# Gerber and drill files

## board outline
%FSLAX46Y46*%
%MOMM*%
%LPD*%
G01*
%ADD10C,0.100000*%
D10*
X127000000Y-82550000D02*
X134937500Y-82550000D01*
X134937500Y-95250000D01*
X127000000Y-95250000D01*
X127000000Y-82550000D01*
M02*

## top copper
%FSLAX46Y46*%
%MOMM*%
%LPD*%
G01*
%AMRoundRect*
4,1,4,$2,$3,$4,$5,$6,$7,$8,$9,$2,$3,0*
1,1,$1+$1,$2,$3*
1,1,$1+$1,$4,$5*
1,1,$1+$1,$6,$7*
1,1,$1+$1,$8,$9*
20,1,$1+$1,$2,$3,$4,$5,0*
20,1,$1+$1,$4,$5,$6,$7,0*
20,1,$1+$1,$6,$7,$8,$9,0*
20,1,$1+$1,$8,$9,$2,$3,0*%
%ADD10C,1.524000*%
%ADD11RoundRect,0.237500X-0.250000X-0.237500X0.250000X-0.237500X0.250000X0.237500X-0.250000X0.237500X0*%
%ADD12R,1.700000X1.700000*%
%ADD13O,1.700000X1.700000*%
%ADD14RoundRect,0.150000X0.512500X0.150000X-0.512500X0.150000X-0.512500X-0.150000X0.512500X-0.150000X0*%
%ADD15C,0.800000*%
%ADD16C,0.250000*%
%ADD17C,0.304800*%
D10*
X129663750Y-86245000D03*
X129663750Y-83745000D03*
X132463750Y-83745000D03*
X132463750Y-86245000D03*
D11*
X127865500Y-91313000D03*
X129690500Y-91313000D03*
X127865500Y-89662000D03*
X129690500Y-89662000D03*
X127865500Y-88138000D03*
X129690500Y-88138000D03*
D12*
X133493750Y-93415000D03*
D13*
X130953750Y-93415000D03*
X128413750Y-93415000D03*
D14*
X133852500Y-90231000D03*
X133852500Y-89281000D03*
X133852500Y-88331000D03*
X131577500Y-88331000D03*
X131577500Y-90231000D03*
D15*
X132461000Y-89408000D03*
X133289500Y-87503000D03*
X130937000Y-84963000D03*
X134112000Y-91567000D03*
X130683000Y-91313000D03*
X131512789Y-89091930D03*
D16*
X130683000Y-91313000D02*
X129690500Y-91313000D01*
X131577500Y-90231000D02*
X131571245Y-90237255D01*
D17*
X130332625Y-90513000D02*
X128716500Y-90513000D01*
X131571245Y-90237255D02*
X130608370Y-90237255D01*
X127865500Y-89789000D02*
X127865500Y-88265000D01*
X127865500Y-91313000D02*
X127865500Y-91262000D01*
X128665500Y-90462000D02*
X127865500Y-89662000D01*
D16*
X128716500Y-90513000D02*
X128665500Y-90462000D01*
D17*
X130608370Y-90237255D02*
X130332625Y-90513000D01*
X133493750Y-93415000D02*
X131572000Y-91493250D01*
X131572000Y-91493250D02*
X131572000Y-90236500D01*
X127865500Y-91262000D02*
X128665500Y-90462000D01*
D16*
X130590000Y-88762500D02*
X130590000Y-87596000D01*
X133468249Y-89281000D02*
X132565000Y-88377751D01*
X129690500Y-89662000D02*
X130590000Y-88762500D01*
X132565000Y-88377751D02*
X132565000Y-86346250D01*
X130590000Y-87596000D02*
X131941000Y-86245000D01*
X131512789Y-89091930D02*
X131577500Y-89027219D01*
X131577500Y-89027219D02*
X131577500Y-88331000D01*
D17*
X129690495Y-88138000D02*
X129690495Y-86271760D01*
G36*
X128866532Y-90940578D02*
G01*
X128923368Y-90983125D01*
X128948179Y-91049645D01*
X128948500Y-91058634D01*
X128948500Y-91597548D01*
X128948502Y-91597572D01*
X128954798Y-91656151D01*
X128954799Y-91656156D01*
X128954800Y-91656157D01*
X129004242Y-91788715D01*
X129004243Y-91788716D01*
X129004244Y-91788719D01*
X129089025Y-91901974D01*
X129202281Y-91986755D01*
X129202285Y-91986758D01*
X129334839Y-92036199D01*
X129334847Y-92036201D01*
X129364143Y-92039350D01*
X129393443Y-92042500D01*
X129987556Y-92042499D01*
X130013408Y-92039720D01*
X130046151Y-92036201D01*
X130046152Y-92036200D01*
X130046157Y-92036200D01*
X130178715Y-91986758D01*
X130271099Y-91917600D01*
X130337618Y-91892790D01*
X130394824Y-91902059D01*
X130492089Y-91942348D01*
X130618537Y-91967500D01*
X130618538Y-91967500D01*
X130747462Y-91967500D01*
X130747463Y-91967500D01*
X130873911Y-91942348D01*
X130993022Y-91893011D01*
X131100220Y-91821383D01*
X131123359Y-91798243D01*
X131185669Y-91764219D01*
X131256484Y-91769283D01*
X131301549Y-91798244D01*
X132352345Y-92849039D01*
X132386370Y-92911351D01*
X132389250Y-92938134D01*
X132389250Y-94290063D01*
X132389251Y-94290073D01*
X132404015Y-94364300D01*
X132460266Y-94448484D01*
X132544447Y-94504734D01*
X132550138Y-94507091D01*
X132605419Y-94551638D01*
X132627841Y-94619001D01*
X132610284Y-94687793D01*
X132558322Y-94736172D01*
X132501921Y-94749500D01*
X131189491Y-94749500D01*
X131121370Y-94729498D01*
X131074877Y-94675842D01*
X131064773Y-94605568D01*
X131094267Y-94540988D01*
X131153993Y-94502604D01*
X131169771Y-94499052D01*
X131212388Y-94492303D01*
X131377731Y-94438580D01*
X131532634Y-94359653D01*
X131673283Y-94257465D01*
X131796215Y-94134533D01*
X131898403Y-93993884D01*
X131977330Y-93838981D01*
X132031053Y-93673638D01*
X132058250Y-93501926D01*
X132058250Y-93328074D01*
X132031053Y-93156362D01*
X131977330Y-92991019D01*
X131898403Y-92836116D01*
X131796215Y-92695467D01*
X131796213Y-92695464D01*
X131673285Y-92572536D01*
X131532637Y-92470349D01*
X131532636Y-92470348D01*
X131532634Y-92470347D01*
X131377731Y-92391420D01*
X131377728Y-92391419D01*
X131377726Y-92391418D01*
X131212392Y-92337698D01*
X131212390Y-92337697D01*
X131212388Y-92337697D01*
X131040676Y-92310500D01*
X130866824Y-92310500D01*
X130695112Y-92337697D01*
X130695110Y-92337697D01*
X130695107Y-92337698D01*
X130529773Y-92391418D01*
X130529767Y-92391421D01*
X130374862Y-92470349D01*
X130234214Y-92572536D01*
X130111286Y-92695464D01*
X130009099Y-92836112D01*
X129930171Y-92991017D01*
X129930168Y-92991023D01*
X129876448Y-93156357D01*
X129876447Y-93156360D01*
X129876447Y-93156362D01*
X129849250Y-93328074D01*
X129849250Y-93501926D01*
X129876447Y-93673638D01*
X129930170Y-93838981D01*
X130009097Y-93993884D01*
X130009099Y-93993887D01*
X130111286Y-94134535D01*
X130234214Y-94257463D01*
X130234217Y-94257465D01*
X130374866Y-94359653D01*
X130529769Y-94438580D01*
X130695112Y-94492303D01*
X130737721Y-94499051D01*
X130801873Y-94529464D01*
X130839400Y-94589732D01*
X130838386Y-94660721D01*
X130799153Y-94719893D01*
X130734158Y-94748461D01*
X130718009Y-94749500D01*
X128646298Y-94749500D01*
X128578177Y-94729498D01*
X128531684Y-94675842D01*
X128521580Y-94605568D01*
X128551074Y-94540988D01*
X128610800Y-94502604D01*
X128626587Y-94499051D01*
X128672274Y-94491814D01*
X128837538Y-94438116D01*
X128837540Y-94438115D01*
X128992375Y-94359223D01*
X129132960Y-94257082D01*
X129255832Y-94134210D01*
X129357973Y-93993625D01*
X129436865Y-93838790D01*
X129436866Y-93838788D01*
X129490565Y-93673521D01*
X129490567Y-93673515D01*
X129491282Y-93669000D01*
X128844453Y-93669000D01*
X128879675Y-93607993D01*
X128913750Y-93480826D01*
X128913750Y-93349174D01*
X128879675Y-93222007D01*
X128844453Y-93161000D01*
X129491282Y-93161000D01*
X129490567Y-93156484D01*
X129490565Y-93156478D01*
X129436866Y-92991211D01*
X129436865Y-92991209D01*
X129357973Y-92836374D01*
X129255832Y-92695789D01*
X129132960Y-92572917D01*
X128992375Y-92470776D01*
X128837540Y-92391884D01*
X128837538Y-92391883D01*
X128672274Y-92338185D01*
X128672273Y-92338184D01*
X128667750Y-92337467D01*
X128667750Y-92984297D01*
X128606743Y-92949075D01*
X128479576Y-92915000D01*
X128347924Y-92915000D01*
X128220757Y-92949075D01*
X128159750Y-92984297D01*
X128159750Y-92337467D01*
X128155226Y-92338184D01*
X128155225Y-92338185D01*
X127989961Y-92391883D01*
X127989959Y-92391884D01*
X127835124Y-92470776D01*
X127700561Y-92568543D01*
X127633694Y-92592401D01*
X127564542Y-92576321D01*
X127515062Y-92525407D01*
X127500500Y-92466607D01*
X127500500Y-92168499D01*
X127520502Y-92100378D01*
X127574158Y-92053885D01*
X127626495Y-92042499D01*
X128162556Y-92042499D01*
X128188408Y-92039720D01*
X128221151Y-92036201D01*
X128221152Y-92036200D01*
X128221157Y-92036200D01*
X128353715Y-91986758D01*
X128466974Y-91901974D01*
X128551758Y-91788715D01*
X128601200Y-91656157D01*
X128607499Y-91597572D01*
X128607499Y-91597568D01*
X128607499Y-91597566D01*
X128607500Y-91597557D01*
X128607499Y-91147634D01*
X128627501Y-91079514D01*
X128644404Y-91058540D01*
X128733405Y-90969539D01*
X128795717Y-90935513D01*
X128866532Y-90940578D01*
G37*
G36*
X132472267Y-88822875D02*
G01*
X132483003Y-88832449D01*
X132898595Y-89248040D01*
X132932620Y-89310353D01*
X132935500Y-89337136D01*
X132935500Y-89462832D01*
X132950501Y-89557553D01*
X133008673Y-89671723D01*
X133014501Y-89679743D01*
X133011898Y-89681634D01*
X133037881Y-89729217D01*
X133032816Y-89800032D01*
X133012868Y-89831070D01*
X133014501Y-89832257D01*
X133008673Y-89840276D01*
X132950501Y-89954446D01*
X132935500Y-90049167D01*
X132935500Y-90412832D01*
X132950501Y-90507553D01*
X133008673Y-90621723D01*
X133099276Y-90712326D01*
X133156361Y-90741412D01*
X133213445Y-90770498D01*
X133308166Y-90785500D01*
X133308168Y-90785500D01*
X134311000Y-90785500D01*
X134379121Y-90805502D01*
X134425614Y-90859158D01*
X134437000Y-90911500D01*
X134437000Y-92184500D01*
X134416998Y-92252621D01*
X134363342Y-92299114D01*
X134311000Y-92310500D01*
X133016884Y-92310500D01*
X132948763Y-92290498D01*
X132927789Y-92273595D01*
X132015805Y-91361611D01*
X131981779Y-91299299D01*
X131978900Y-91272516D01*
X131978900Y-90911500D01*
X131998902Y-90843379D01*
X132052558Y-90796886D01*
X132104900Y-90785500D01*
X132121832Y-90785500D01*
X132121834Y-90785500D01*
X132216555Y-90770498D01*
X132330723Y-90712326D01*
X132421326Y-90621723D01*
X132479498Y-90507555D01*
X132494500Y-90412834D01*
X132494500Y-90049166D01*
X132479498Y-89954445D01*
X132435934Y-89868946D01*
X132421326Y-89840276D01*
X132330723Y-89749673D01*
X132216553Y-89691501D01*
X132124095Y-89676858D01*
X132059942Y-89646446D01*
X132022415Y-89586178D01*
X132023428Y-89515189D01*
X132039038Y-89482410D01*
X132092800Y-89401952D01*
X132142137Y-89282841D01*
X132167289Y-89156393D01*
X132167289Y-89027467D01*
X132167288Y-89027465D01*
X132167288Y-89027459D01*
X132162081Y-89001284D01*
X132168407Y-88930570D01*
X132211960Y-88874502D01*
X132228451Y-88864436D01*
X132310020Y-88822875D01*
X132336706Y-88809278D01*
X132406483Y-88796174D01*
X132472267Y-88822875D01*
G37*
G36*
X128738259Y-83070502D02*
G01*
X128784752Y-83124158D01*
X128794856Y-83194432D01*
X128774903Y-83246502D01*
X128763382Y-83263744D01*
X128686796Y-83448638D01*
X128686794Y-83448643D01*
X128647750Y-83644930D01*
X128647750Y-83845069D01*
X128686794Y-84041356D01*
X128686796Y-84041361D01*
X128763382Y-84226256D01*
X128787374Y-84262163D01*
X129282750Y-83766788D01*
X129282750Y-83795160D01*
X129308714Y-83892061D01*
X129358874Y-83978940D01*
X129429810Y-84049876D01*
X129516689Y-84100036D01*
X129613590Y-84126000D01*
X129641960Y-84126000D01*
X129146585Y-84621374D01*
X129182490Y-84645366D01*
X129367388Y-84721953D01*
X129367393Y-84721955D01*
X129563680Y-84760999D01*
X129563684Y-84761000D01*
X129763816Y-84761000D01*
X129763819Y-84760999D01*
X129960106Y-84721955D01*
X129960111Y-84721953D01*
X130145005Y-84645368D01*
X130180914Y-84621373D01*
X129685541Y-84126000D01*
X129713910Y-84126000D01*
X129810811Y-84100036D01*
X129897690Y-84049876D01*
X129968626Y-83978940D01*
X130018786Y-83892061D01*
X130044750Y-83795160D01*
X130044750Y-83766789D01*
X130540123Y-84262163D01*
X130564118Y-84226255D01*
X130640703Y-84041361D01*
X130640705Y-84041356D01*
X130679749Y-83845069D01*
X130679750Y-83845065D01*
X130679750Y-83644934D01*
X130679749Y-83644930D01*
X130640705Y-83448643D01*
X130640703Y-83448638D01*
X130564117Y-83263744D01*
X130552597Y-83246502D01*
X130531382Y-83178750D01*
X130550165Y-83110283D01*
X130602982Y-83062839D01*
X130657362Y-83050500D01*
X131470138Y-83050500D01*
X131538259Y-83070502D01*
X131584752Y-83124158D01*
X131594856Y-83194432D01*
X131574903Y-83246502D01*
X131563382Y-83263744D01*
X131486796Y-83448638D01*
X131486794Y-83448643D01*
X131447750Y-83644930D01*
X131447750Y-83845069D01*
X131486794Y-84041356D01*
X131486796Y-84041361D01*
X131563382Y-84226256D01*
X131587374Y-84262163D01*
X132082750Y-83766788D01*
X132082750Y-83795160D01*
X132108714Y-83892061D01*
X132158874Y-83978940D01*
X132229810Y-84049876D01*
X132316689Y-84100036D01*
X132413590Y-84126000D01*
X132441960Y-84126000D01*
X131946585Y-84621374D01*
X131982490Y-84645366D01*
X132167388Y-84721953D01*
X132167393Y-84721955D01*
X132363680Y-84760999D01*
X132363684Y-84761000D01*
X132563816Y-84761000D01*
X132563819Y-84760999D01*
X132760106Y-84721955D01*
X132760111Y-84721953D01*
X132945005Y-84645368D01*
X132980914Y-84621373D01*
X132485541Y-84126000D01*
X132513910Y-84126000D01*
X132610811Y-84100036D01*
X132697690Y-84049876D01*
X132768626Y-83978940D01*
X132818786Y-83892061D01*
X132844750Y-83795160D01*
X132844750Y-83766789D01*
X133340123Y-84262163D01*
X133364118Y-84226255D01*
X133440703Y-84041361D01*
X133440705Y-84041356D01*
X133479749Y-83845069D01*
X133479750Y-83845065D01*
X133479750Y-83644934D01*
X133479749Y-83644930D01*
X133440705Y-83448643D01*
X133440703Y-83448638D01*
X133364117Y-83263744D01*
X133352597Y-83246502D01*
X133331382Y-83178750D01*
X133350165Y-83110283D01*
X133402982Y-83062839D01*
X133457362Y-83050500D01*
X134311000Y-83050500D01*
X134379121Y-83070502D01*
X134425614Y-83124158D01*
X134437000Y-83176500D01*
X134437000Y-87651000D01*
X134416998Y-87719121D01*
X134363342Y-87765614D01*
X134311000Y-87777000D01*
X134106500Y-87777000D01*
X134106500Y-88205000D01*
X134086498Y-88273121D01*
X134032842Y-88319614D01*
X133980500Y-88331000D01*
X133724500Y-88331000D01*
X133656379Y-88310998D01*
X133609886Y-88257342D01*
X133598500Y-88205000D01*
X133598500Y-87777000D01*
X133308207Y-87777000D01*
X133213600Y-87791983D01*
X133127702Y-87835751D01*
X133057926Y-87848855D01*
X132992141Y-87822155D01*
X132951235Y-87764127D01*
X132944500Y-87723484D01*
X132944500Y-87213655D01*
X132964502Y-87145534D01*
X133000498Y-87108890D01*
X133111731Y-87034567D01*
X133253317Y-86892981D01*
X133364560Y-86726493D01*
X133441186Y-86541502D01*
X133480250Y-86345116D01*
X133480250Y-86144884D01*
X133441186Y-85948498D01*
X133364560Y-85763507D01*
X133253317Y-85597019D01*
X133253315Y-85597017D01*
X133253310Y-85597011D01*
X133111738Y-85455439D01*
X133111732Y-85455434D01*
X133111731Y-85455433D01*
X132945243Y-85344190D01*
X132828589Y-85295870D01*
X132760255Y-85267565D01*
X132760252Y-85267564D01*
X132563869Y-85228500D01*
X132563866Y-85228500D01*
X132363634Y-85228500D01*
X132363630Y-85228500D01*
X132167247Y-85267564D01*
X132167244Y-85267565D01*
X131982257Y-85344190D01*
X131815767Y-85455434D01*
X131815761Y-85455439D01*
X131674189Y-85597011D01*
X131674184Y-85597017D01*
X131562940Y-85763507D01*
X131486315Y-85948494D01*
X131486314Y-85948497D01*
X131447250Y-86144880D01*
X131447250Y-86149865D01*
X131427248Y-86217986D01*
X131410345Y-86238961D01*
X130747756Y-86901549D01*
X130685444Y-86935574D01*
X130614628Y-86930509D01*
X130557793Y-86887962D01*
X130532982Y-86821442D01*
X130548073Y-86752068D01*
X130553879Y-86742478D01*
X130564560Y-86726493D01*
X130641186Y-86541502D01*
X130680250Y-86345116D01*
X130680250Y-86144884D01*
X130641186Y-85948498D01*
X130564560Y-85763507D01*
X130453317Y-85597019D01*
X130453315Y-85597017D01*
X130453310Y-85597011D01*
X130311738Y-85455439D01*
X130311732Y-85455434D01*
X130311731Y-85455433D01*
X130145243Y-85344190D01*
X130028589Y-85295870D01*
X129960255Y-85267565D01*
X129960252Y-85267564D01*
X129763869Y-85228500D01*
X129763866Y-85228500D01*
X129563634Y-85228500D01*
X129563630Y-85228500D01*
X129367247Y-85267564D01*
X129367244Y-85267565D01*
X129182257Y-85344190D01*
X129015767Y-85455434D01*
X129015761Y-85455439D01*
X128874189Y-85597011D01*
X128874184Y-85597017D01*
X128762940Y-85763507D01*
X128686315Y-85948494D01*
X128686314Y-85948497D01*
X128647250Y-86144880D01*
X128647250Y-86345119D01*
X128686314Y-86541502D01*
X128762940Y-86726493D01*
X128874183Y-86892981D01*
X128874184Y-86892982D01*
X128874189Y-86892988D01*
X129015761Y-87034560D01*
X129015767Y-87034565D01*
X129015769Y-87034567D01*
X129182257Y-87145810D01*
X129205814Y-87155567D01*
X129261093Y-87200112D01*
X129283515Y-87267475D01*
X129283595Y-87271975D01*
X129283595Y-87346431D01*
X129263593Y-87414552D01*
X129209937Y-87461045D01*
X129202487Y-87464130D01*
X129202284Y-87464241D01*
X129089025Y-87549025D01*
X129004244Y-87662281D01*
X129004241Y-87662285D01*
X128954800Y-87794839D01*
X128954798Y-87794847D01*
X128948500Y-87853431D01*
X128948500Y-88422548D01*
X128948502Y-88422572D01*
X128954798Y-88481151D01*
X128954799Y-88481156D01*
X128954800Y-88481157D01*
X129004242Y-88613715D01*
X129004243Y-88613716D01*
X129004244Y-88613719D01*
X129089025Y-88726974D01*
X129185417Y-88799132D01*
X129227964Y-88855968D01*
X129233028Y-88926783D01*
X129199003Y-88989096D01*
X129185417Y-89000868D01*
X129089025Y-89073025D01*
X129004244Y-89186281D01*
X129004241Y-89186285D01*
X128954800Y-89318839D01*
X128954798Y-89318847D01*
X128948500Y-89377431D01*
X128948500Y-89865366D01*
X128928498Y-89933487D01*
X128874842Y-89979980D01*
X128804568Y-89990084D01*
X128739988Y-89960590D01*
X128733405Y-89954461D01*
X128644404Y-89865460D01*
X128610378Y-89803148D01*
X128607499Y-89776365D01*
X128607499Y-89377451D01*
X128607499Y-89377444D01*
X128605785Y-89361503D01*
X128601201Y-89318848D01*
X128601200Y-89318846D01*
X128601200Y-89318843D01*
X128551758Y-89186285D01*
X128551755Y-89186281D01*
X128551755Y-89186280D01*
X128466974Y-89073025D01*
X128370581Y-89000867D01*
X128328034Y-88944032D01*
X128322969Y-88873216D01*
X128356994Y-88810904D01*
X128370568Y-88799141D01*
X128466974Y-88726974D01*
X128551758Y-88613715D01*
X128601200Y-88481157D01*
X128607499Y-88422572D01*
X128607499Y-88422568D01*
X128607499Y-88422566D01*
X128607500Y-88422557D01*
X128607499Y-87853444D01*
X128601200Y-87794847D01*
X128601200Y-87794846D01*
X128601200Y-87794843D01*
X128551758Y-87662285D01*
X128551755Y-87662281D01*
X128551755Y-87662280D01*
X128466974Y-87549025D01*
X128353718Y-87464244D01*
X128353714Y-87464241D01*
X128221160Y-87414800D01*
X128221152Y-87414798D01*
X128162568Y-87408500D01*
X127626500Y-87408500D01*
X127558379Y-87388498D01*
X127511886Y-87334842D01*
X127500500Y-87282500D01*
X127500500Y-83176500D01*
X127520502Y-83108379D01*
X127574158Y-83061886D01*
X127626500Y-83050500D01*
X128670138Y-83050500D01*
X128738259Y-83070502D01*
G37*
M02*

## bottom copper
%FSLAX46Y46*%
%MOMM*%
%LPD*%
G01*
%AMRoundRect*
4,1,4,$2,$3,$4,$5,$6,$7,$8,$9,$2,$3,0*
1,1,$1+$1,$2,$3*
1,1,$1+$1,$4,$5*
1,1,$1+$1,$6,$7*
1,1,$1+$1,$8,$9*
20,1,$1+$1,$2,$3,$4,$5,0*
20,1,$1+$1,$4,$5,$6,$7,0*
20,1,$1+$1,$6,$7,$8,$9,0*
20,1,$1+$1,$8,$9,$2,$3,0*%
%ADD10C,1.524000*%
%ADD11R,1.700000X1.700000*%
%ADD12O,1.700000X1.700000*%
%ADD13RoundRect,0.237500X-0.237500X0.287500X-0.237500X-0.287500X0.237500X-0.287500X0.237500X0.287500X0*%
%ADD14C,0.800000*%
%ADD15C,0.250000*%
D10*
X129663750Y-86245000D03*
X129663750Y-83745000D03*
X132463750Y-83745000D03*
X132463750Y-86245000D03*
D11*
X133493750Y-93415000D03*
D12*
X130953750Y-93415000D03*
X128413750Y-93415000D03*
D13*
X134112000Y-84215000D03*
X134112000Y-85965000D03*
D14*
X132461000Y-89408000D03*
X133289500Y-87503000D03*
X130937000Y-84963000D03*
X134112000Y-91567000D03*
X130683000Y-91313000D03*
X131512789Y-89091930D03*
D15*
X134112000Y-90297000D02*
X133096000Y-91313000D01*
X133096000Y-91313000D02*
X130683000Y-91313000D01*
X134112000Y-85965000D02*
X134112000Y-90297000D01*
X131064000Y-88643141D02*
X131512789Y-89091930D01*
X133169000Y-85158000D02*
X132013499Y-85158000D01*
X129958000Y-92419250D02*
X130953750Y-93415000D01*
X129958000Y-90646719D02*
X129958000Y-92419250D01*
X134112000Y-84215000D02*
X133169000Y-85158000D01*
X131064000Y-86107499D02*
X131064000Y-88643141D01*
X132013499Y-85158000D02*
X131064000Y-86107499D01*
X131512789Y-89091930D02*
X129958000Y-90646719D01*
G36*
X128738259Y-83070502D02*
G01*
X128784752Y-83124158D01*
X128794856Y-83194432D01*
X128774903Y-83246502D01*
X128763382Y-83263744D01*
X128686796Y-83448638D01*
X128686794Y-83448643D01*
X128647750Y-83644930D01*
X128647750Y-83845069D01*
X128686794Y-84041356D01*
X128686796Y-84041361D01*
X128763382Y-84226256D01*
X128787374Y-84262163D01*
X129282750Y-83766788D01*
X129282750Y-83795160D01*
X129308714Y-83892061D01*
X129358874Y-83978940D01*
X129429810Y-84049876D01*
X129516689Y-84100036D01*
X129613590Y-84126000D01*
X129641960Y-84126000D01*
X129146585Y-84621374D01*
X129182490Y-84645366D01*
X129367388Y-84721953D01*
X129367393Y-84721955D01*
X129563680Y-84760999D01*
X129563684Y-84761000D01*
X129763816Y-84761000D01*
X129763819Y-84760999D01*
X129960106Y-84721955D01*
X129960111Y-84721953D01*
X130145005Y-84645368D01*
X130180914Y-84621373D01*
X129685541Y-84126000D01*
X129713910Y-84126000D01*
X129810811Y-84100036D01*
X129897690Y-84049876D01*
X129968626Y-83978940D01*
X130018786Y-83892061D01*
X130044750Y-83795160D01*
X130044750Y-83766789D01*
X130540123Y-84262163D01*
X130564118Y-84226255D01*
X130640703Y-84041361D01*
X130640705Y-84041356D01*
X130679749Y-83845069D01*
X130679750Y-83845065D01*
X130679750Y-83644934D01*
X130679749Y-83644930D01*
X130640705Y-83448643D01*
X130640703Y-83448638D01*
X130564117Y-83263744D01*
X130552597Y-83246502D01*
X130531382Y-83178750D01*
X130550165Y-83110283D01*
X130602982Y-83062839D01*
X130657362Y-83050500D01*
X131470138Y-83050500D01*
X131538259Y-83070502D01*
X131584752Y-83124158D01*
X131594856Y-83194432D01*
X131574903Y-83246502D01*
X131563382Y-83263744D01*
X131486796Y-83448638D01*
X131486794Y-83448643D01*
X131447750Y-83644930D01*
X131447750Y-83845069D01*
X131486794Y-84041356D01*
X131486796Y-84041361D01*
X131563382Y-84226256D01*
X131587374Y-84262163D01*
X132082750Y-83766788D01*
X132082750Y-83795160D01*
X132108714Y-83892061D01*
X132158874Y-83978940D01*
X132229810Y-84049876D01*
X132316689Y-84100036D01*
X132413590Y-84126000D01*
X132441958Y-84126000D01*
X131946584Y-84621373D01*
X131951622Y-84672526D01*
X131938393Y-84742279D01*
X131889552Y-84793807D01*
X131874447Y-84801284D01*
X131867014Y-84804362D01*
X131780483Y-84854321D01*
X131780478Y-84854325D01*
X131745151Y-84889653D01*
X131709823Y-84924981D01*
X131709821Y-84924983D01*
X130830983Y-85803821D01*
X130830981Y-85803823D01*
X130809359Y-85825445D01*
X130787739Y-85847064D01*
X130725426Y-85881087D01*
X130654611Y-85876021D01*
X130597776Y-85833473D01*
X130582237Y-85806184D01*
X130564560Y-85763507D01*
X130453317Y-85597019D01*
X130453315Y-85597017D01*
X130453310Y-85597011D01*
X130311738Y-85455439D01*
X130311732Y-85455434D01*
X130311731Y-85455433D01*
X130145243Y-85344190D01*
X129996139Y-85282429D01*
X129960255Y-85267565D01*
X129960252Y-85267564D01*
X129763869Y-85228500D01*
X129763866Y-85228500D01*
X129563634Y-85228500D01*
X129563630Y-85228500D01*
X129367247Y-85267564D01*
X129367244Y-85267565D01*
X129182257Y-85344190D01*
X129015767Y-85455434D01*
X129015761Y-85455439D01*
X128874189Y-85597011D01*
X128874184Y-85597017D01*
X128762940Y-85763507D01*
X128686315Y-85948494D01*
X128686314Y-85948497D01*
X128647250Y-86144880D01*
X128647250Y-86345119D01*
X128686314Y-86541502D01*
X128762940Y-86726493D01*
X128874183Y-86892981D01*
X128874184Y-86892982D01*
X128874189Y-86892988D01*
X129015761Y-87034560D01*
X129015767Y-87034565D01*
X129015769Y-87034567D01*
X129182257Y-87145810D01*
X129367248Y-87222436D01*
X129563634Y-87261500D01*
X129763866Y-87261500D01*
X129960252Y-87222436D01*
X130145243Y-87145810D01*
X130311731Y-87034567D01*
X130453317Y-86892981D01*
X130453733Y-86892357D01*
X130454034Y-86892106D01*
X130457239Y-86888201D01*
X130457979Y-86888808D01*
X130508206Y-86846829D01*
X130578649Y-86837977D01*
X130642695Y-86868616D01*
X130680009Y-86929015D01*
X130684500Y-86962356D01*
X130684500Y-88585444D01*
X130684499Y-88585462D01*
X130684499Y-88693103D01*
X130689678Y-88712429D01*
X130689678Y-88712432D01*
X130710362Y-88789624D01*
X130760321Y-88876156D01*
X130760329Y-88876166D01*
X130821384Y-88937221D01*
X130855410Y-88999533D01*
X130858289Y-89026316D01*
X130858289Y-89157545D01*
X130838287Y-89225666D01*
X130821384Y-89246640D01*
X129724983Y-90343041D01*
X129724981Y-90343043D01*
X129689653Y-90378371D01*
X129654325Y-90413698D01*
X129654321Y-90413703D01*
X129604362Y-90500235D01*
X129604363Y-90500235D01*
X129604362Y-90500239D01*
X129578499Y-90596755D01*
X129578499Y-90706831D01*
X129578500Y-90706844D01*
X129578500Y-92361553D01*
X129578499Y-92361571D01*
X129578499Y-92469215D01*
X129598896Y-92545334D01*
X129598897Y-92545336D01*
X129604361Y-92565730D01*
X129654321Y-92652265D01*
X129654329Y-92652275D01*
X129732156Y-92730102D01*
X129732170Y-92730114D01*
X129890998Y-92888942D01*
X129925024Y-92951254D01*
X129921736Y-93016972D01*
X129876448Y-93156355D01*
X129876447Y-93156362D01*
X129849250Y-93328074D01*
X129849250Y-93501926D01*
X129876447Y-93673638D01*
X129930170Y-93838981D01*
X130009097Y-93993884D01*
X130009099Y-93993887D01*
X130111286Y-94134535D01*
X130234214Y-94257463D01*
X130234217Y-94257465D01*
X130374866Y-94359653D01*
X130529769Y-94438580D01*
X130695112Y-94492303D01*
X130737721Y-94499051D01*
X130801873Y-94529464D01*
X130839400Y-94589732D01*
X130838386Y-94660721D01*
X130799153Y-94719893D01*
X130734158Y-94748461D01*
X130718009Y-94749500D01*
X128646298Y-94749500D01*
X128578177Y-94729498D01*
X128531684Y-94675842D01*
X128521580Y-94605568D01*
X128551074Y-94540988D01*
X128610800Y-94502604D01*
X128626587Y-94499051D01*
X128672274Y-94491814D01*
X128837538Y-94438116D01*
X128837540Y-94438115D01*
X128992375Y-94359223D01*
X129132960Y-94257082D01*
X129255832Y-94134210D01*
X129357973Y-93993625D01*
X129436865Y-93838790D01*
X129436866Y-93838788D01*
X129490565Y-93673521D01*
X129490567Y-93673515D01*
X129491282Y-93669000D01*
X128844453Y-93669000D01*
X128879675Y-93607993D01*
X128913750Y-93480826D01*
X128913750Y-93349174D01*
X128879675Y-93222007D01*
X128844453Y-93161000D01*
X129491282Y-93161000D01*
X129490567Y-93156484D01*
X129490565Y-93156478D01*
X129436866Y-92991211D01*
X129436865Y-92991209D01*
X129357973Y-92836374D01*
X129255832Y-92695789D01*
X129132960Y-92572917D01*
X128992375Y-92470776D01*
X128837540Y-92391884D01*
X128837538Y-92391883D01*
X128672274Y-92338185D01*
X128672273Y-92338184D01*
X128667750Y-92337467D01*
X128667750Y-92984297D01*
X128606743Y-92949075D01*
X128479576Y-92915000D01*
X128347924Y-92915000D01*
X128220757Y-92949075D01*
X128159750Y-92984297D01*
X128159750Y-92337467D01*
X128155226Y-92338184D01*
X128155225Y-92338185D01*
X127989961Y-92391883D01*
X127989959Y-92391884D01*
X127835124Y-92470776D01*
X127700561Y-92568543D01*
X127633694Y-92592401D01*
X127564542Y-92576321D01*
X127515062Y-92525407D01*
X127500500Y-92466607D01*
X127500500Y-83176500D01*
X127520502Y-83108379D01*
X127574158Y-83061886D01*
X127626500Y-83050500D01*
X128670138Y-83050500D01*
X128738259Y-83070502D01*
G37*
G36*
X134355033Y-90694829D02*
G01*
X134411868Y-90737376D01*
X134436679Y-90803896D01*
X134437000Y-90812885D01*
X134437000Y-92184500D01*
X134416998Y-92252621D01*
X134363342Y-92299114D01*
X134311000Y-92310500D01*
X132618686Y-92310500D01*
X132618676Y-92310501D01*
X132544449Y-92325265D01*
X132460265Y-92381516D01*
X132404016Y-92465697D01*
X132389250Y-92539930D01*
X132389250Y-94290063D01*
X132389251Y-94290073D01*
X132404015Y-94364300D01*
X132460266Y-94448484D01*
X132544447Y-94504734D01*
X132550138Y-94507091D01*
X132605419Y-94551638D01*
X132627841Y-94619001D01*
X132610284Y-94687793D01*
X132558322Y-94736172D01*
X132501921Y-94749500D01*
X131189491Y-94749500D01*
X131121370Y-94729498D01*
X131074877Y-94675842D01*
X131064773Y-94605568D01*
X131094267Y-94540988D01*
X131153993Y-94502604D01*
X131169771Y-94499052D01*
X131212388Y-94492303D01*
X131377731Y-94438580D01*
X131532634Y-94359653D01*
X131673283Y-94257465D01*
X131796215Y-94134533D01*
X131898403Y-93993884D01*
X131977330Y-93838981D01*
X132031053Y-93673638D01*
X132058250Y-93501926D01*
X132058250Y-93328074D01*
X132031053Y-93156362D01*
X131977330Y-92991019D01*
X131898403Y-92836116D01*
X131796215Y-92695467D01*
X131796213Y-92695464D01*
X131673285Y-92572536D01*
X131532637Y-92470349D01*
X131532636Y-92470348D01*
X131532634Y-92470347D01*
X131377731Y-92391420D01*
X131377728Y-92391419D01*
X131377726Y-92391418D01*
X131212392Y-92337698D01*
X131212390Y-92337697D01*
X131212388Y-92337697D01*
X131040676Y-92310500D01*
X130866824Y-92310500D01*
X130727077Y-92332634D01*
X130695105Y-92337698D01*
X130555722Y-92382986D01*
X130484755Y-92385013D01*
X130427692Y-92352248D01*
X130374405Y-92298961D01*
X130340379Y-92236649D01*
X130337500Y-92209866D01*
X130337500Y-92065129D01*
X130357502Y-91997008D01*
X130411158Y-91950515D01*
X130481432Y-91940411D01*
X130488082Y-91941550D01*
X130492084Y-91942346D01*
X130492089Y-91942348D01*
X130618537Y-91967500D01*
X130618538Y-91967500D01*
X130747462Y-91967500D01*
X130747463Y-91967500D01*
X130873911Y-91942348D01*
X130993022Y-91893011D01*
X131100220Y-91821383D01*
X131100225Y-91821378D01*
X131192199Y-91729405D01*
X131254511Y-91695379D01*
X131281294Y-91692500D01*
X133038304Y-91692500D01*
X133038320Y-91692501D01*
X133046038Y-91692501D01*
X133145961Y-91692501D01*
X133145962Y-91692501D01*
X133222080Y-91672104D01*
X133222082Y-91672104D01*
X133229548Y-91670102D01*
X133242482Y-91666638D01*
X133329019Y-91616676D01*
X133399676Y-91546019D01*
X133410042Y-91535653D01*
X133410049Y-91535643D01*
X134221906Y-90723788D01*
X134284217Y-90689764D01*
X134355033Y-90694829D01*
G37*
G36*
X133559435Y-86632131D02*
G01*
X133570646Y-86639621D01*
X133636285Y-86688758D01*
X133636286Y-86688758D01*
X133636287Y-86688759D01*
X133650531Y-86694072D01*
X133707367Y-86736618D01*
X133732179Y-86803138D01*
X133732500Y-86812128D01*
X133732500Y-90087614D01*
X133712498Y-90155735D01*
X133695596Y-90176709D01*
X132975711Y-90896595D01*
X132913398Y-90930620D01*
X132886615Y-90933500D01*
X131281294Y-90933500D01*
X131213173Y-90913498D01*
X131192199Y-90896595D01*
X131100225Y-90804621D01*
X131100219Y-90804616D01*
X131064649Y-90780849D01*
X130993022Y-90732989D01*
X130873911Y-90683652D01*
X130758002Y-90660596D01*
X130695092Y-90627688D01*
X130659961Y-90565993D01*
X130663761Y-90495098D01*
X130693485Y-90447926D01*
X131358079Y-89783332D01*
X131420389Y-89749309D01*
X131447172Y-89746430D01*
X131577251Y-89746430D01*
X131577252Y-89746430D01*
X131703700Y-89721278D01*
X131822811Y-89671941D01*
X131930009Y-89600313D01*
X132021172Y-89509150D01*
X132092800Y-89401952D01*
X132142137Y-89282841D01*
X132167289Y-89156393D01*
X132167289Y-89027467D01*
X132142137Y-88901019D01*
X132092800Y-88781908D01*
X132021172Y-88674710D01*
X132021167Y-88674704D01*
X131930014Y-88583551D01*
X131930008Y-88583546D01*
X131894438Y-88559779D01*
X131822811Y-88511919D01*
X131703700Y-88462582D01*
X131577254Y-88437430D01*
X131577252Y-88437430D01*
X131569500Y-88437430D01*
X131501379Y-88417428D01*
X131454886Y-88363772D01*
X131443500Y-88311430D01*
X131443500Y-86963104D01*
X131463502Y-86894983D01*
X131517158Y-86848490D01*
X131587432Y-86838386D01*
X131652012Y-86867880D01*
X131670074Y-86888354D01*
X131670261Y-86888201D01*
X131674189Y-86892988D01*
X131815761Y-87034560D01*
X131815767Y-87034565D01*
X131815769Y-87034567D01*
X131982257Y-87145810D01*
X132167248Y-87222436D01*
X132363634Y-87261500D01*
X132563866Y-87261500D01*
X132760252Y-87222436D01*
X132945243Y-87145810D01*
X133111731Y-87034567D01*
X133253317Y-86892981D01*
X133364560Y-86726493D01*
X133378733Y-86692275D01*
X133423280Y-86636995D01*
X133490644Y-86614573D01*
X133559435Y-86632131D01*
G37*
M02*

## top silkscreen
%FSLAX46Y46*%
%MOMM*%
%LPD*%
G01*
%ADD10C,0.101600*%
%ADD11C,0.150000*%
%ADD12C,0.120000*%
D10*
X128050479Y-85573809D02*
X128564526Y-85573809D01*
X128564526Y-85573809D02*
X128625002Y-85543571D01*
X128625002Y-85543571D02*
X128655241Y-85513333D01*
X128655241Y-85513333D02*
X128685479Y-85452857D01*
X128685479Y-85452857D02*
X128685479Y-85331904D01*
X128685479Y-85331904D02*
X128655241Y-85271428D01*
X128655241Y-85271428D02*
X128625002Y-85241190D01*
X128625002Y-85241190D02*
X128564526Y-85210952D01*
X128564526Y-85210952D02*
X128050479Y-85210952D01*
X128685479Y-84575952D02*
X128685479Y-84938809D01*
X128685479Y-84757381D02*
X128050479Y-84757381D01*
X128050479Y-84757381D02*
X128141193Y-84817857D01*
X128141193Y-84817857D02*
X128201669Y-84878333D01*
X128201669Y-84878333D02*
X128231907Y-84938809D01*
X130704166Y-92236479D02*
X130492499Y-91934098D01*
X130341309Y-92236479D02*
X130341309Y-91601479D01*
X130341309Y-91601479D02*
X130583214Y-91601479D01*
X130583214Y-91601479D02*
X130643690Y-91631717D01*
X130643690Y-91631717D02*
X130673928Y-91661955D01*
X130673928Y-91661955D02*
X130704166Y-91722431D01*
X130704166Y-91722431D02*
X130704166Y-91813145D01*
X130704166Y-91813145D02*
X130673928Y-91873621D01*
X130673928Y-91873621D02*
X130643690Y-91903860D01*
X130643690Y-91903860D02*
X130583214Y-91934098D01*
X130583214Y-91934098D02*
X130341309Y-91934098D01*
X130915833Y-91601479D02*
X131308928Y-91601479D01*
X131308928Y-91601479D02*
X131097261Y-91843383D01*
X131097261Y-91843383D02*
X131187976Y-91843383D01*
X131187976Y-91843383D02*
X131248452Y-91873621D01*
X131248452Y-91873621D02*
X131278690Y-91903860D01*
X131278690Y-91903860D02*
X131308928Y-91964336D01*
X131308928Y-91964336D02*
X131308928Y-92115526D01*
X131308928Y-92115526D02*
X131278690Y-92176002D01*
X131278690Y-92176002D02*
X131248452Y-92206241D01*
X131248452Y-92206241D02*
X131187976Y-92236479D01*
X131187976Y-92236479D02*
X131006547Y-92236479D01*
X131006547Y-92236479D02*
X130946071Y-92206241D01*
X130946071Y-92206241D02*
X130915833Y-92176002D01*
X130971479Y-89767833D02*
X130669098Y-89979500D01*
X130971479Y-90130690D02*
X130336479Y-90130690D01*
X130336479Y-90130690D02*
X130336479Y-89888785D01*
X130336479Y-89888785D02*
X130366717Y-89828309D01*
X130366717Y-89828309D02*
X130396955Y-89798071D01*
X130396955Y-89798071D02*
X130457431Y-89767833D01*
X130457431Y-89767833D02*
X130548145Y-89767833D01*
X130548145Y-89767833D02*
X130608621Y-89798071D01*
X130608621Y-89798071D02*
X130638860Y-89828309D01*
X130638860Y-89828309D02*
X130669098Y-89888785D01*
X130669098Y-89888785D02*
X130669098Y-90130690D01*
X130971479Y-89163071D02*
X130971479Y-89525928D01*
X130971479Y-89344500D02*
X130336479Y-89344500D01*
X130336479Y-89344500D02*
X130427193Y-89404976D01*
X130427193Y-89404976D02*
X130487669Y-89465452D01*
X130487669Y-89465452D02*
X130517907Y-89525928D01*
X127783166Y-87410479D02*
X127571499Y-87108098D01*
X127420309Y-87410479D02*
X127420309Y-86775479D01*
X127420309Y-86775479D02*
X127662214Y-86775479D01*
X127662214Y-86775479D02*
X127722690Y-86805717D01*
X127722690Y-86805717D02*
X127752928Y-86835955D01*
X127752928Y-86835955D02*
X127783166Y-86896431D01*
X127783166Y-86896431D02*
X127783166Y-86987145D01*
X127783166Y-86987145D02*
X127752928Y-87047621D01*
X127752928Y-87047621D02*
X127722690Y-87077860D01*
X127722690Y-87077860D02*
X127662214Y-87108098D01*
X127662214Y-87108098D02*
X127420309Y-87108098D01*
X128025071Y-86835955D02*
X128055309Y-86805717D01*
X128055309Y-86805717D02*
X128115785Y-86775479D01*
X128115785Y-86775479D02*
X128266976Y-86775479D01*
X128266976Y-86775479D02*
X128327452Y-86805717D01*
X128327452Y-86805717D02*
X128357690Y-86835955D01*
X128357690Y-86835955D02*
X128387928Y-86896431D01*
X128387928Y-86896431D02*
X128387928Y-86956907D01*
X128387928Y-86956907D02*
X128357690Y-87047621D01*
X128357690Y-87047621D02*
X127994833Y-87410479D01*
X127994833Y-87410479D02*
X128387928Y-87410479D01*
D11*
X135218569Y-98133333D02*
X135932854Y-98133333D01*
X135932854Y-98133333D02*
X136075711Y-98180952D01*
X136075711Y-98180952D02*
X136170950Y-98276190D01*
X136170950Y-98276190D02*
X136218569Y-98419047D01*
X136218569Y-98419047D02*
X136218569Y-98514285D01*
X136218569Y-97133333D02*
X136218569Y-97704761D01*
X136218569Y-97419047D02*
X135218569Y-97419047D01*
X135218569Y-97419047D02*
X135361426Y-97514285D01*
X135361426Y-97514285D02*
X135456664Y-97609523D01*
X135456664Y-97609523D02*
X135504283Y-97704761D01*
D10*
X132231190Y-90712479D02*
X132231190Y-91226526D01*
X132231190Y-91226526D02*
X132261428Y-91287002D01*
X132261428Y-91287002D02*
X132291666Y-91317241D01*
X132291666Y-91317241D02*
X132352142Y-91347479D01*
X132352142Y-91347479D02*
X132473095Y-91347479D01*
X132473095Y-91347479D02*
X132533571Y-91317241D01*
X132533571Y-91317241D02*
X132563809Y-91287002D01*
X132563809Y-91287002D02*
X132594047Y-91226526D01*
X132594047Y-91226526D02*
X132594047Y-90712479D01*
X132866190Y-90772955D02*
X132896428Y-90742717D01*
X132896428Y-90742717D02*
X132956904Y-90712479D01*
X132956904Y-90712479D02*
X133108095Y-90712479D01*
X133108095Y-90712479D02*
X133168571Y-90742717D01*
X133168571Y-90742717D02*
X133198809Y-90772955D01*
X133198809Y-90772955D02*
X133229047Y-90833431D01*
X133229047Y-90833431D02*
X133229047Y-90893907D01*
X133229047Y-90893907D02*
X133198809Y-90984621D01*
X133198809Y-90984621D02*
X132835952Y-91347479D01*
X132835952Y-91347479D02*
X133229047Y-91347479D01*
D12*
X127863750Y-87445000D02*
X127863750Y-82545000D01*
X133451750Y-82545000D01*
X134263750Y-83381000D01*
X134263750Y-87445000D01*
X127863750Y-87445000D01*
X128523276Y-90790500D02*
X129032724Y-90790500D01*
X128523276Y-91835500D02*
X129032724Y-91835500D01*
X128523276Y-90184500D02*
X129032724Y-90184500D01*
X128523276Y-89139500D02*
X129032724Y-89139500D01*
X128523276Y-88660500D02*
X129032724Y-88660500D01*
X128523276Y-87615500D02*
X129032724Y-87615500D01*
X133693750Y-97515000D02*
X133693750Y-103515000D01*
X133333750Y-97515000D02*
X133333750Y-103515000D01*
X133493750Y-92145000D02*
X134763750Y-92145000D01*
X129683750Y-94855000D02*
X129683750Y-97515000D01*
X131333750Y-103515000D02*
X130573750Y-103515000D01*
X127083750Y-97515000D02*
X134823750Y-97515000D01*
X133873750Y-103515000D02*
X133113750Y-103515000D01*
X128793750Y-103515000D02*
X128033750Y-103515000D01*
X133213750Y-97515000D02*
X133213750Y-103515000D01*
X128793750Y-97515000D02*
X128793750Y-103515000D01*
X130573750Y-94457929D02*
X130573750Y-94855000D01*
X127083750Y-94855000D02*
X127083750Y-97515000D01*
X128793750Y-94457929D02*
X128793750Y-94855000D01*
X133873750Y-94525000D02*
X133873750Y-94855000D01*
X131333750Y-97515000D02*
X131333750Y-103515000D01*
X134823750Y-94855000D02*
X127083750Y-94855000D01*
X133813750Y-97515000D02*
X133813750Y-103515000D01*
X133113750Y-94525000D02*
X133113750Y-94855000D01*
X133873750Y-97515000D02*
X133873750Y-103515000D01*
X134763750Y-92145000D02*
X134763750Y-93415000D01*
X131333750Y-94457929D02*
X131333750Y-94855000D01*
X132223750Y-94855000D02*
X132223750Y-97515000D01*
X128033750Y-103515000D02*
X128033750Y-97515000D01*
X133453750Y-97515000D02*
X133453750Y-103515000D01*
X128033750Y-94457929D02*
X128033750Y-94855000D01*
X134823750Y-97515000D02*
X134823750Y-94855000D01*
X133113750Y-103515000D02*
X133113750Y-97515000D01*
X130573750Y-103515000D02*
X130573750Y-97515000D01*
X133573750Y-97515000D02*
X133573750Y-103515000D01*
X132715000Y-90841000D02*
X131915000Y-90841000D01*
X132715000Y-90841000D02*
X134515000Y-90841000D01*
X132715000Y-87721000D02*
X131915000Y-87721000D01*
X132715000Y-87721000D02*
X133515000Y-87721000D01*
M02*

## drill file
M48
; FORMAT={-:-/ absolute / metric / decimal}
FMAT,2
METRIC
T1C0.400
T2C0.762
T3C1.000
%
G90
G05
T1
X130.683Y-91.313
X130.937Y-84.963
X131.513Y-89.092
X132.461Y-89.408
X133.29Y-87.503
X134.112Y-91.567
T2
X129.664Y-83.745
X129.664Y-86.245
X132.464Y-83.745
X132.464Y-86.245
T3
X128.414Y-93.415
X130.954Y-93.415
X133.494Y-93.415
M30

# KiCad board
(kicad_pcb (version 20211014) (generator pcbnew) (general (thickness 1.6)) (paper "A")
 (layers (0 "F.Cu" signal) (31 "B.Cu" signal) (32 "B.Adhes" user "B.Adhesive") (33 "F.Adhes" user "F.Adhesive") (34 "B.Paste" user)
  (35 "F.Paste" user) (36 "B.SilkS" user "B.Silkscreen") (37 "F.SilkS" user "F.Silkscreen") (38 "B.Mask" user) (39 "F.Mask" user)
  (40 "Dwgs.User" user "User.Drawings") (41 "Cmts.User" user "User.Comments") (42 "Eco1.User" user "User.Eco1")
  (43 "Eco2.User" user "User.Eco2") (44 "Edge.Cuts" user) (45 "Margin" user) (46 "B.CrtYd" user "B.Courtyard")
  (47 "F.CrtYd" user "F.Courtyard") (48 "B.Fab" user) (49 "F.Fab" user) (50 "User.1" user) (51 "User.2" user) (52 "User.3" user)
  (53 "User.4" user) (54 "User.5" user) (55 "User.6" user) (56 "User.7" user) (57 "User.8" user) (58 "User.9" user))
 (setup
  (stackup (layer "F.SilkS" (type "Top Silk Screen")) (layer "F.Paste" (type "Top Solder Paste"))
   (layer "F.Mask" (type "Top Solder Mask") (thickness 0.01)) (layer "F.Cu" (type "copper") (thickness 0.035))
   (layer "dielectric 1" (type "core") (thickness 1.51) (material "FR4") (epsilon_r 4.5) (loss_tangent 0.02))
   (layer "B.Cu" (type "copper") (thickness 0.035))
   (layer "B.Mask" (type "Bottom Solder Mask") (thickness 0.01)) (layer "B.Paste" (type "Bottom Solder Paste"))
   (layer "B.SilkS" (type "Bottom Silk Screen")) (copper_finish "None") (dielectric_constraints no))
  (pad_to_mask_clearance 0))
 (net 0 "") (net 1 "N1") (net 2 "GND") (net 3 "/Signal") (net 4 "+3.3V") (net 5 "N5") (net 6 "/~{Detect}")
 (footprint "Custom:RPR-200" (layer "F.Cu") (at 127.86375 87.445)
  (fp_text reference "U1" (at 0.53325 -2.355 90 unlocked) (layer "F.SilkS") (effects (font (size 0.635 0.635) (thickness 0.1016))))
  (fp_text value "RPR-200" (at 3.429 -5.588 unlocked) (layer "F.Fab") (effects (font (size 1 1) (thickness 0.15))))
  (fp_poly (pts (xy 0 0) (xy 0 -4.9) (xy 5.588 -4.9) (xy 6.4 -4.064) (xy 6.4 0)) (layer "F.SilkS") (width 0.12) (fill none))
  (pad "1" thru_hole circle (at 1.8 -1.2) (size 1.524 1.524) (drill 0.762) (layers *.Cu *.Mask) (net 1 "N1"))
  (pad "2" thru_hole circle (at 1.8 -3.7) (size 1.524 1.524) (drill 0.762) (layers *.Cu *.Mask) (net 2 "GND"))
  (pad "3" thru_hole circle (at 4.6 -3.7) (size 1.524 1.524) (drill 0.762) (layers *.Cu *.Mask) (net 2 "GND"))
  (pad "4" thru_hole circle (at 4.6 -1.2) (size 1.524 1.524) (drill 0.762) (layers *.Cu *.Mask) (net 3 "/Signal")))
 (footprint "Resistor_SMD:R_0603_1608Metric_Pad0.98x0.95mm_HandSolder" (layer "F.Cu") (at 128.778 91.313)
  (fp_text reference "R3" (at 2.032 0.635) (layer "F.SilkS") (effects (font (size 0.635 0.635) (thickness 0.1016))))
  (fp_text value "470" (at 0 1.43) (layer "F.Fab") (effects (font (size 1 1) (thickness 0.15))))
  (fp_line (start -0.254724 -0.5225) (end 0.254724 -0.5225) (layer "F.SilkS") (width 0.12))
  (fp_line (start -0.254724 0.5225) (end 0.254724 0.5225) (layer "F.SilkS") (width 0.12))
  (pad "1" smd roundrect (at -0.9125 0) (size 0.975 0.95) (layers "F.Cu" "F.Paste" "F.Mask") (roundrect_rratio 0.25) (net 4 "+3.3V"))
  (pad "2" smd roundrect (at 0.9125 0) (size 0.975 0.95) (layers "F.Cu" "F.Paste" "F.Mask") (roundrect_rratio 0.25) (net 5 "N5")))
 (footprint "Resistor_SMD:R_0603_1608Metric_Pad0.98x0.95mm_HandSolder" (layer "F.Cu") (at 128.778 89.662)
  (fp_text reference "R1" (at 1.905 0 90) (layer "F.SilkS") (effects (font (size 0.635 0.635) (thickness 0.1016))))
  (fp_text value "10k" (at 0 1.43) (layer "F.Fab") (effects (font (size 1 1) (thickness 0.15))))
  (fp_line (start -0.254724 0.5225) (end 0.254724 0.5225) (layer "F.SilkS") (width 0.12))
  (fp_line (start -0.254724 -0.5225) (end 0.254724 -0.5225) (layer "F.SilkS") (width 0.12))
  (pad "1" smd roundrect (at -0.9125 0) (size 0.975 0.95) (layers "F.Cu" "F.Paste" "F.Mask") (roundrect_rratio 0.25) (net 4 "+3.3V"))
  (pad "2" smd roundrect (at 0.9125 0) (size 0.975 0.95) (layers "F.Cu" "F.Paste" "F.Mask") (roundrect_rratio 0.25) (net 3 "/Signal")))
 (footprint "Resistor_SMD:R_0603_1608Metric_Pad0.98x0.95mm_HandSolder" (layer "F.Cu") (at 128.778 88.138)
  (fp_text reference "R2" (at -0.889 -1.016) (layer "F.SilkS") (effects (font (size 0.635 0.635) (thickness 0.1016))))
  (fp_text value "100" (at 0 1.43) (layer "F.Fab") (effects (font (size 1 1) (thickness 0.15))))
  (fp_line (start -0.254724 0.5225) (end 0.254724 0.5225) (layer "F.SilkS") (width 0.12))
  (fp_line (start -0.254724 -0.5225) (end 0.254724 -0.5225) (layer "F.SilkS") (width 0.12))
  (pad "1" smd roundrect (at -0.9125 0) (size 0.975 0.95) (layers "F.Cu" "F.Paste" "F.Mask") (roundrect_rratio 0.25) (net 4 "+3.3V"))
  (pad "2" smd roundrect (at 0.9125 0) (size 0.975 0.95) (layers "F.Cu" "F.Paste" "F.Mask") (roundrect_rratio 0.25) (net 1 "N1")))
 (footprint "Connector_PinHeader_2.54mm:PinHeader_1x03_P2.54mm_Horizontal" (layer "F.Cu") (at 133.49375 93.415 -90)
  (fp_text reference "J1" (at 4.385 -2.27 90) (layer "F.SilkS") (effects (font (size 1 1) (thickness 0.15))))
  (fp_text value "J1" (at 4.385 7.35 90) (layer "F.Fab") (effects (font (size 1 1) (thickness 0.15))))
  (fp_line (start 4.1 -0.2) (end 10.1 -0.2) (layer "F.SilkS") (width 0.12))
  (fp_line (start 4.1 0.16) (end 10.1 0.16) (layer "F.SilkS") (width 0.12))
  (fp_line (start -1.27 0) (end -1.27 -1.27) (layer "F.SilkS") (width 0.12))
  (fp_line (start 1.44 3.81) (end 4.1 3.81) (layer "F.SilkS") (width 0.12))
  (fp_line (start 10.1 2.16) (end 10.1 2.92) (layer "F.SilkS") (width 0.12))
  (fp_line (start 4.1 6.41) (end 4.1 -1.33) (layer "F.SilkS") (width 0.12))
  (fp_line (start 10.1 -0.38) (end 10.1 0.38) (layer "F.SilkS") (width 0.12))
  (fp_line (start 10.1 4.7) (end 10.1 5.46) (layer "F.SilkS") (width 0.12))
  (fp_line (start 4.1 0.28) (end 10.1 0.28) (layer "F.SilkS") (width 0.12))
  (fp_line (start 4.1 4.7) (end 10.1 4.7) (layer "F.SilkS") (width 0.12))
  (fp_line (start 1.042929 2.92) (end 1.44 2.92) (layer "F.SilkS") (width 0.12))
  (fp_line (start 1.44 6.41) (end 4.1 6.41) (layer "F.SilkS") (width 0.12))
  (fp_line (start 1.042929 4.7) (end 1.44 4.7) (layer "F.SilkS") (width 0.12))
  (fp_line (start 1.11 -0.38) (end 1.44 -0.38) (layer "F.SilkS") (width 0.12))
  (fp_line (start 4.1 2.16) (end 10.1 2.16) (layer "F.SilkS") (width 0.12))
  (fp_line (start 1.44 -1.33) (end 1.44 6.41) (layer "F.SilkS") (width 0.12))
  (fp_line (start 4.1 -0.32) (end 10.1 -0.32) (layer "F.SilkS") (width 0.12))
  (fp_line (start 1.11 0.38) (end 1.44 0.38) (layer "F.SilkS") (width 0.12))
  (fp_line (start 4.1 -0.38) (end 10.1 -0.38) (layer "F.SilkS") (width 0.12))
  (fp_line (start -1.27 -1.27) (end 0 -1.27) (layer "F.SilkS") (width 0.12))
  (fp_line (start 1.042929 2.16) (end 1.44 2.16) (layer "F.SilkS") (width 0.12))
  (fp_line (start 1.44 1.27) (end 4.1 1.27) (layer "F.SilkS") (width 0.12))
  (fp_line (start 10.1 5.46) (end 4.1 5.46) (layer "F.SilkS") (width 0.12))
  (fp_line (start 4.1 0.04) (end 10.1 0.04) (layer "F.SilkS") (width 0.12))
  (fp_line (start 1.042929 5.46) (end 1.44 5.46) (layer "F.SilkS") (width 0.12))
  (fp_line (start 4.1 -1.33) (end 1.44 -1.33) (layer "F.SilkS") (width 0.12))
  (fp_line (start 10.1 0.38) (end 4.1 0.38) (layer "F.SilkS") (width 0.12))
  (fp_line (start 10.1 2.92) (end 4.1 2.92) (layer "F.SilkS") (width 0.12))
  (fp_line (start 4.1 -0.08) (end 10.1 -0.08) (layer "F.SilkS") (width 0.12))
  (pad "1" thru_hole rect (at 0 0 270) (size 1.7 1.7) (drill 1) (layers *.Cu *.Mask) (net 4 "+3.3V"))
  (pad "2" thru_hole oval (at 0 2.54 270) (size 1.7 1.7) (drill 1) (layers *.Cu *.Mask) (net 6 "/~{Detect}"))
  (pad "3" thru_hole oval (at 0 5.08 270) (size 1.7 1.7) (drill 1) (layers *.Cu *.Mask) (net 2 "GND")))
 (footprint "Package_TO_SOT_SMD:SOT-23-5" (layer "F.Cu") (at 132.715 89.281 180)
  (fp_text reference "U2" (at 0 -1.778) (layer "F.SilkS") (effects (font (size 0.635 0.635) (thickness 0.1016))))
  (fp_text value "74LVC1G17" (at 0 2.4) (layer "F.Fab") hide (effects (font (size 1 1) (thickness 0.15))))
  (fp_line (start 0 -1.56) (end 0.8 -1.56) (layer "F.SilkS") (width 0.12))
  (fp_line (start 0 -1.56) (end -1.8 -1.56) (layer "F.SilkS") (width 0.12))
  (fp_line (start 0 1.56) (end 0.8 1.56) (layer "F.SilkS") (width 0.12))
  (fp_line (start 0 1.56) (end -0.8 1.56) (layer "F.SilkS") (width 0.12))
  (pad "1" smd roundrect (at -1.1375 -0.95 180) (size 1.325 0.6) (layers "F.Cu" "F.Paste" "F.Mask") (roundrect_rratio 0.25))
  (pad "2" smd roundrect (at -1.1375 0 180) (size 1.325 0.6) (layers "F.Cu" "F.Paste" "F.Mask") (roundrect_rratio 0.25) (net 3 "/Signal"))
  (pad "3" smd roundrect (at -1.1375 0.95 180) (size 1.325 0.6) (layers "F.Cu" "F.Paste" "F.Mask") (roundrect_rratio 0.25) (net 2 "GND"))
  (pad "4" smd roundrect (at 1.1375 0.95 180) (size 1.325 0.6) (layers "F.Cu" "F.Paste" "F.Mask") (roundrect_rratio 0.25)
   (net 6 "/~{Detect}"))
  (pad "5" smd roundrect (at 1.1375 -0.95 180) (size 1.325 0.6) (layers "F.Cu" "F.Paste" "F.Mask") (roundrect_rratio 0.25) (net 4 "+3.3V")))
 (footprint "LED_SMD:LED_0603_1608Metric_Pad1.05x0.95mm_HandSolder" (layer "B.Cu") (at 134.112 85.09 -90)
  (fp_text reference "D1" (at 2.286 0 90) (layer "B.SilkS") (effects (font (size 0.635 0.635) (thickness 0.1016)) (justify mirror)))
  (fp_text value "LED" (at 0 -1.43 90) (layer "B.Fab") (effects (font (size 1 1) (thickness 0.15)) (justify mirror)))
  (pad "1" smd roundrect (at -0.875 0 270) (size 1.05 0.95) (layers "B.Cu" "B.Paste" "B.Mask") (roundrect_rratio 0.25) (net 6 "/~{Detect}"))
  (pad "2" smd roundrect (at 0.875 0 270) (size 1.05 0.95) (layers "B.Cu" "B.Paste" "B.Mask") (roundrect_rratio 0.25) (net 5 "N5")))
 (gr_rect (start 127 82.55) (end 134.9375 95.25) (layer "Edge.Cuts") (width 0.1) (fill none))
 (via (at 132.461 89.408) (size 0.8) (drill 0.4) (layers "F.Cu" "B.Cu") (free) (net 2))
 (via (at 133.2895 87.503) (size 0.8) (drill 0.4) (layers "F.Cu" "B.Cu") (free) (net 2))
 (via (at 130.937 84.963) (size 0.8) (drill 0.4) (layers "F.Cu" "B.Cu") (free) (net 2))
 (via (at 134.112 91.567) (size 0.8) (drill 0.4) (layers "F.Cu" "B.Cu") (free) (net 2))
 (segment (start 130.683 91.313) (end 129.6905 91.313) (width 0.25) (layer "F.Cu") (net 5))
 (via (at 130.683 91.313) (size 0.8) (drill 0.4) (layers "F.Cu" "B.Cu") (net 5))
 (segment (start 134.112 90.297) (end 133.096 91.313) (width 0.25) (layer "B.Cu") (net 5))
 (segment (start 133.096 91.313) (end 130.683 91.313) (width 0.25) (layer "B.Cu") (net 5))
 (segment (start 134.112 85.965) (end 134.112 90.297) (width 0.25) (layer "B.Cu") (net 5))
 (segment (start 131.5775 90.231) (end 131.571245 90.237255) (width 0.25) (layer "F.Cu") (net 4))
 (segment (start 130.332625 90.513) (end 128.7165 90.513) (width 0.3048) (layer "F.Cu") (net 4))
 (segment (start 131.571245 90.237255) (end 130.60837 90.237255) (width 0.3048) (layer "F.Cu") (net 4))
 (segment (start 127.8655 89.789) (end 127.8655 88.265) (width 0.3048) (layer "F.Cu") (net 4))
 (segment (start 127.8655 91.313) (end 127.8655 91.262) (width 0.3048) (layer "F.Cu") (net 4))
 (segment (start 128.6655 90.462) (end 127.8655 89.662) (width 0.3048) (layer "F.Cu") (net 4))
 (segment (start 128.7165 90.513) (end 128.6655 90.462) (width 0.25) (layer "F.Cu") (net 4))
 (segment (start 130.60837 90.237255) (end 130.332625 90.513) (width 0.3048) (layer "F.Cu") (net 4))
 (segment (start 133.49375 93.415) (end 131.572 91.49325) (width 0.3048) (layer "F.Cu") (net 4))
 (segment (start 131.572 91.49325) (end 131.572 90.2365) (width 0.3048) (layer "F.Cu") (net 4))
 (segment (start 127.8655 91.262) (end 128.6655 90.462) (width 0.3048) (layer "F.Cu") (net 4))
 (segment (start 130.59 88.7625) (end 130.59 87.596) (width 0.25) (layer "F.Cu") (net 3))
 (segment (start 133.468249 89.281) (end 132.565 88.377751) (width 0.25) (layer "F.Cu") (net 3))
 (segment (start 129.6905 89.662) (end 130.59 88.7625) (width 0.25) (layer "F.Cu") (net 3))
 (segment (start 132.565 88.377751) (end 132.565 86.34625) (width 0.25) (layer "F.Cu") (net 3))
 (segment (start 130.59 87.596) (end 131.941 86.245) (width 0.25) (layer "F.Cu") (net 3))
 (segment (start 131.512789 89.09193) (end 131.5775 89.027219) (width 0.25) (layer "F.Cu") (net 6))
 (segment (start 131.5775 89.027219) (end 131.5775 88.331) (width 0.25) (layer "F.Cu") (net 6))
 (via (at 131.512789 89.09193) (size 0.8) (drill 0.4) (layers "F.Cu" "B.Cu") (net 6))
 (segment (start 131.064 88.643141) (end 131.512789 89.09193) (width 0.25) (layer "B.Cu") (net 6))
 (segment (start 133.169 85.158) (end 132.013499 85.158) (width 0.25) (layer "B.Cu") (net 6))
 (segment (start 129.958 92.41925) (end 130.95375 93.415) (width 0.25) (layer "B.Cu") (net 6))
 (segment (start 129.958 90.646719) (end 129.958 92.41925) (width 0.25) (layer "B.Cu") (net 6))
 (segment (start 134.112 84.215) (end 133.169 85.158) (width 0.25) (layer "B.Cu") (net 6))
 (segment (start 131.064 86.107499) (end 131.064 88.643141) (width 0.25) (layer "B.Cu") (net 6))
 (segment (start 132.013499 85.158) (end 131.064 86.107499) (width 0.25) (layer "B.Cu") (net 6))
 (segment (start 131.512789 89.09193) (end 129.958 90.646719) (width 0.25) (layer "B.Cu") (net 6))
 (segment (start 129.690495 88.138) (end 129.690495 86.27176) (width 0.3048) (layer "F.Cu") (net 1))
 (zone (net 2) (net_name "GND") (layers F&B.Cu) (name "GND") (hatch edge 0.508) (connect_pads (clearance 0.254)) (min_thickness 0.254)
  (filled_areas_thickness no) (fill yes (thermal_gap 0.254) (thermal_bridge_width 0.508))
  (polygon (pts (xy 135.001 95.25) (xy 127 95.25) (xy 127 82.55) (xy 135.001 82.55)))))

